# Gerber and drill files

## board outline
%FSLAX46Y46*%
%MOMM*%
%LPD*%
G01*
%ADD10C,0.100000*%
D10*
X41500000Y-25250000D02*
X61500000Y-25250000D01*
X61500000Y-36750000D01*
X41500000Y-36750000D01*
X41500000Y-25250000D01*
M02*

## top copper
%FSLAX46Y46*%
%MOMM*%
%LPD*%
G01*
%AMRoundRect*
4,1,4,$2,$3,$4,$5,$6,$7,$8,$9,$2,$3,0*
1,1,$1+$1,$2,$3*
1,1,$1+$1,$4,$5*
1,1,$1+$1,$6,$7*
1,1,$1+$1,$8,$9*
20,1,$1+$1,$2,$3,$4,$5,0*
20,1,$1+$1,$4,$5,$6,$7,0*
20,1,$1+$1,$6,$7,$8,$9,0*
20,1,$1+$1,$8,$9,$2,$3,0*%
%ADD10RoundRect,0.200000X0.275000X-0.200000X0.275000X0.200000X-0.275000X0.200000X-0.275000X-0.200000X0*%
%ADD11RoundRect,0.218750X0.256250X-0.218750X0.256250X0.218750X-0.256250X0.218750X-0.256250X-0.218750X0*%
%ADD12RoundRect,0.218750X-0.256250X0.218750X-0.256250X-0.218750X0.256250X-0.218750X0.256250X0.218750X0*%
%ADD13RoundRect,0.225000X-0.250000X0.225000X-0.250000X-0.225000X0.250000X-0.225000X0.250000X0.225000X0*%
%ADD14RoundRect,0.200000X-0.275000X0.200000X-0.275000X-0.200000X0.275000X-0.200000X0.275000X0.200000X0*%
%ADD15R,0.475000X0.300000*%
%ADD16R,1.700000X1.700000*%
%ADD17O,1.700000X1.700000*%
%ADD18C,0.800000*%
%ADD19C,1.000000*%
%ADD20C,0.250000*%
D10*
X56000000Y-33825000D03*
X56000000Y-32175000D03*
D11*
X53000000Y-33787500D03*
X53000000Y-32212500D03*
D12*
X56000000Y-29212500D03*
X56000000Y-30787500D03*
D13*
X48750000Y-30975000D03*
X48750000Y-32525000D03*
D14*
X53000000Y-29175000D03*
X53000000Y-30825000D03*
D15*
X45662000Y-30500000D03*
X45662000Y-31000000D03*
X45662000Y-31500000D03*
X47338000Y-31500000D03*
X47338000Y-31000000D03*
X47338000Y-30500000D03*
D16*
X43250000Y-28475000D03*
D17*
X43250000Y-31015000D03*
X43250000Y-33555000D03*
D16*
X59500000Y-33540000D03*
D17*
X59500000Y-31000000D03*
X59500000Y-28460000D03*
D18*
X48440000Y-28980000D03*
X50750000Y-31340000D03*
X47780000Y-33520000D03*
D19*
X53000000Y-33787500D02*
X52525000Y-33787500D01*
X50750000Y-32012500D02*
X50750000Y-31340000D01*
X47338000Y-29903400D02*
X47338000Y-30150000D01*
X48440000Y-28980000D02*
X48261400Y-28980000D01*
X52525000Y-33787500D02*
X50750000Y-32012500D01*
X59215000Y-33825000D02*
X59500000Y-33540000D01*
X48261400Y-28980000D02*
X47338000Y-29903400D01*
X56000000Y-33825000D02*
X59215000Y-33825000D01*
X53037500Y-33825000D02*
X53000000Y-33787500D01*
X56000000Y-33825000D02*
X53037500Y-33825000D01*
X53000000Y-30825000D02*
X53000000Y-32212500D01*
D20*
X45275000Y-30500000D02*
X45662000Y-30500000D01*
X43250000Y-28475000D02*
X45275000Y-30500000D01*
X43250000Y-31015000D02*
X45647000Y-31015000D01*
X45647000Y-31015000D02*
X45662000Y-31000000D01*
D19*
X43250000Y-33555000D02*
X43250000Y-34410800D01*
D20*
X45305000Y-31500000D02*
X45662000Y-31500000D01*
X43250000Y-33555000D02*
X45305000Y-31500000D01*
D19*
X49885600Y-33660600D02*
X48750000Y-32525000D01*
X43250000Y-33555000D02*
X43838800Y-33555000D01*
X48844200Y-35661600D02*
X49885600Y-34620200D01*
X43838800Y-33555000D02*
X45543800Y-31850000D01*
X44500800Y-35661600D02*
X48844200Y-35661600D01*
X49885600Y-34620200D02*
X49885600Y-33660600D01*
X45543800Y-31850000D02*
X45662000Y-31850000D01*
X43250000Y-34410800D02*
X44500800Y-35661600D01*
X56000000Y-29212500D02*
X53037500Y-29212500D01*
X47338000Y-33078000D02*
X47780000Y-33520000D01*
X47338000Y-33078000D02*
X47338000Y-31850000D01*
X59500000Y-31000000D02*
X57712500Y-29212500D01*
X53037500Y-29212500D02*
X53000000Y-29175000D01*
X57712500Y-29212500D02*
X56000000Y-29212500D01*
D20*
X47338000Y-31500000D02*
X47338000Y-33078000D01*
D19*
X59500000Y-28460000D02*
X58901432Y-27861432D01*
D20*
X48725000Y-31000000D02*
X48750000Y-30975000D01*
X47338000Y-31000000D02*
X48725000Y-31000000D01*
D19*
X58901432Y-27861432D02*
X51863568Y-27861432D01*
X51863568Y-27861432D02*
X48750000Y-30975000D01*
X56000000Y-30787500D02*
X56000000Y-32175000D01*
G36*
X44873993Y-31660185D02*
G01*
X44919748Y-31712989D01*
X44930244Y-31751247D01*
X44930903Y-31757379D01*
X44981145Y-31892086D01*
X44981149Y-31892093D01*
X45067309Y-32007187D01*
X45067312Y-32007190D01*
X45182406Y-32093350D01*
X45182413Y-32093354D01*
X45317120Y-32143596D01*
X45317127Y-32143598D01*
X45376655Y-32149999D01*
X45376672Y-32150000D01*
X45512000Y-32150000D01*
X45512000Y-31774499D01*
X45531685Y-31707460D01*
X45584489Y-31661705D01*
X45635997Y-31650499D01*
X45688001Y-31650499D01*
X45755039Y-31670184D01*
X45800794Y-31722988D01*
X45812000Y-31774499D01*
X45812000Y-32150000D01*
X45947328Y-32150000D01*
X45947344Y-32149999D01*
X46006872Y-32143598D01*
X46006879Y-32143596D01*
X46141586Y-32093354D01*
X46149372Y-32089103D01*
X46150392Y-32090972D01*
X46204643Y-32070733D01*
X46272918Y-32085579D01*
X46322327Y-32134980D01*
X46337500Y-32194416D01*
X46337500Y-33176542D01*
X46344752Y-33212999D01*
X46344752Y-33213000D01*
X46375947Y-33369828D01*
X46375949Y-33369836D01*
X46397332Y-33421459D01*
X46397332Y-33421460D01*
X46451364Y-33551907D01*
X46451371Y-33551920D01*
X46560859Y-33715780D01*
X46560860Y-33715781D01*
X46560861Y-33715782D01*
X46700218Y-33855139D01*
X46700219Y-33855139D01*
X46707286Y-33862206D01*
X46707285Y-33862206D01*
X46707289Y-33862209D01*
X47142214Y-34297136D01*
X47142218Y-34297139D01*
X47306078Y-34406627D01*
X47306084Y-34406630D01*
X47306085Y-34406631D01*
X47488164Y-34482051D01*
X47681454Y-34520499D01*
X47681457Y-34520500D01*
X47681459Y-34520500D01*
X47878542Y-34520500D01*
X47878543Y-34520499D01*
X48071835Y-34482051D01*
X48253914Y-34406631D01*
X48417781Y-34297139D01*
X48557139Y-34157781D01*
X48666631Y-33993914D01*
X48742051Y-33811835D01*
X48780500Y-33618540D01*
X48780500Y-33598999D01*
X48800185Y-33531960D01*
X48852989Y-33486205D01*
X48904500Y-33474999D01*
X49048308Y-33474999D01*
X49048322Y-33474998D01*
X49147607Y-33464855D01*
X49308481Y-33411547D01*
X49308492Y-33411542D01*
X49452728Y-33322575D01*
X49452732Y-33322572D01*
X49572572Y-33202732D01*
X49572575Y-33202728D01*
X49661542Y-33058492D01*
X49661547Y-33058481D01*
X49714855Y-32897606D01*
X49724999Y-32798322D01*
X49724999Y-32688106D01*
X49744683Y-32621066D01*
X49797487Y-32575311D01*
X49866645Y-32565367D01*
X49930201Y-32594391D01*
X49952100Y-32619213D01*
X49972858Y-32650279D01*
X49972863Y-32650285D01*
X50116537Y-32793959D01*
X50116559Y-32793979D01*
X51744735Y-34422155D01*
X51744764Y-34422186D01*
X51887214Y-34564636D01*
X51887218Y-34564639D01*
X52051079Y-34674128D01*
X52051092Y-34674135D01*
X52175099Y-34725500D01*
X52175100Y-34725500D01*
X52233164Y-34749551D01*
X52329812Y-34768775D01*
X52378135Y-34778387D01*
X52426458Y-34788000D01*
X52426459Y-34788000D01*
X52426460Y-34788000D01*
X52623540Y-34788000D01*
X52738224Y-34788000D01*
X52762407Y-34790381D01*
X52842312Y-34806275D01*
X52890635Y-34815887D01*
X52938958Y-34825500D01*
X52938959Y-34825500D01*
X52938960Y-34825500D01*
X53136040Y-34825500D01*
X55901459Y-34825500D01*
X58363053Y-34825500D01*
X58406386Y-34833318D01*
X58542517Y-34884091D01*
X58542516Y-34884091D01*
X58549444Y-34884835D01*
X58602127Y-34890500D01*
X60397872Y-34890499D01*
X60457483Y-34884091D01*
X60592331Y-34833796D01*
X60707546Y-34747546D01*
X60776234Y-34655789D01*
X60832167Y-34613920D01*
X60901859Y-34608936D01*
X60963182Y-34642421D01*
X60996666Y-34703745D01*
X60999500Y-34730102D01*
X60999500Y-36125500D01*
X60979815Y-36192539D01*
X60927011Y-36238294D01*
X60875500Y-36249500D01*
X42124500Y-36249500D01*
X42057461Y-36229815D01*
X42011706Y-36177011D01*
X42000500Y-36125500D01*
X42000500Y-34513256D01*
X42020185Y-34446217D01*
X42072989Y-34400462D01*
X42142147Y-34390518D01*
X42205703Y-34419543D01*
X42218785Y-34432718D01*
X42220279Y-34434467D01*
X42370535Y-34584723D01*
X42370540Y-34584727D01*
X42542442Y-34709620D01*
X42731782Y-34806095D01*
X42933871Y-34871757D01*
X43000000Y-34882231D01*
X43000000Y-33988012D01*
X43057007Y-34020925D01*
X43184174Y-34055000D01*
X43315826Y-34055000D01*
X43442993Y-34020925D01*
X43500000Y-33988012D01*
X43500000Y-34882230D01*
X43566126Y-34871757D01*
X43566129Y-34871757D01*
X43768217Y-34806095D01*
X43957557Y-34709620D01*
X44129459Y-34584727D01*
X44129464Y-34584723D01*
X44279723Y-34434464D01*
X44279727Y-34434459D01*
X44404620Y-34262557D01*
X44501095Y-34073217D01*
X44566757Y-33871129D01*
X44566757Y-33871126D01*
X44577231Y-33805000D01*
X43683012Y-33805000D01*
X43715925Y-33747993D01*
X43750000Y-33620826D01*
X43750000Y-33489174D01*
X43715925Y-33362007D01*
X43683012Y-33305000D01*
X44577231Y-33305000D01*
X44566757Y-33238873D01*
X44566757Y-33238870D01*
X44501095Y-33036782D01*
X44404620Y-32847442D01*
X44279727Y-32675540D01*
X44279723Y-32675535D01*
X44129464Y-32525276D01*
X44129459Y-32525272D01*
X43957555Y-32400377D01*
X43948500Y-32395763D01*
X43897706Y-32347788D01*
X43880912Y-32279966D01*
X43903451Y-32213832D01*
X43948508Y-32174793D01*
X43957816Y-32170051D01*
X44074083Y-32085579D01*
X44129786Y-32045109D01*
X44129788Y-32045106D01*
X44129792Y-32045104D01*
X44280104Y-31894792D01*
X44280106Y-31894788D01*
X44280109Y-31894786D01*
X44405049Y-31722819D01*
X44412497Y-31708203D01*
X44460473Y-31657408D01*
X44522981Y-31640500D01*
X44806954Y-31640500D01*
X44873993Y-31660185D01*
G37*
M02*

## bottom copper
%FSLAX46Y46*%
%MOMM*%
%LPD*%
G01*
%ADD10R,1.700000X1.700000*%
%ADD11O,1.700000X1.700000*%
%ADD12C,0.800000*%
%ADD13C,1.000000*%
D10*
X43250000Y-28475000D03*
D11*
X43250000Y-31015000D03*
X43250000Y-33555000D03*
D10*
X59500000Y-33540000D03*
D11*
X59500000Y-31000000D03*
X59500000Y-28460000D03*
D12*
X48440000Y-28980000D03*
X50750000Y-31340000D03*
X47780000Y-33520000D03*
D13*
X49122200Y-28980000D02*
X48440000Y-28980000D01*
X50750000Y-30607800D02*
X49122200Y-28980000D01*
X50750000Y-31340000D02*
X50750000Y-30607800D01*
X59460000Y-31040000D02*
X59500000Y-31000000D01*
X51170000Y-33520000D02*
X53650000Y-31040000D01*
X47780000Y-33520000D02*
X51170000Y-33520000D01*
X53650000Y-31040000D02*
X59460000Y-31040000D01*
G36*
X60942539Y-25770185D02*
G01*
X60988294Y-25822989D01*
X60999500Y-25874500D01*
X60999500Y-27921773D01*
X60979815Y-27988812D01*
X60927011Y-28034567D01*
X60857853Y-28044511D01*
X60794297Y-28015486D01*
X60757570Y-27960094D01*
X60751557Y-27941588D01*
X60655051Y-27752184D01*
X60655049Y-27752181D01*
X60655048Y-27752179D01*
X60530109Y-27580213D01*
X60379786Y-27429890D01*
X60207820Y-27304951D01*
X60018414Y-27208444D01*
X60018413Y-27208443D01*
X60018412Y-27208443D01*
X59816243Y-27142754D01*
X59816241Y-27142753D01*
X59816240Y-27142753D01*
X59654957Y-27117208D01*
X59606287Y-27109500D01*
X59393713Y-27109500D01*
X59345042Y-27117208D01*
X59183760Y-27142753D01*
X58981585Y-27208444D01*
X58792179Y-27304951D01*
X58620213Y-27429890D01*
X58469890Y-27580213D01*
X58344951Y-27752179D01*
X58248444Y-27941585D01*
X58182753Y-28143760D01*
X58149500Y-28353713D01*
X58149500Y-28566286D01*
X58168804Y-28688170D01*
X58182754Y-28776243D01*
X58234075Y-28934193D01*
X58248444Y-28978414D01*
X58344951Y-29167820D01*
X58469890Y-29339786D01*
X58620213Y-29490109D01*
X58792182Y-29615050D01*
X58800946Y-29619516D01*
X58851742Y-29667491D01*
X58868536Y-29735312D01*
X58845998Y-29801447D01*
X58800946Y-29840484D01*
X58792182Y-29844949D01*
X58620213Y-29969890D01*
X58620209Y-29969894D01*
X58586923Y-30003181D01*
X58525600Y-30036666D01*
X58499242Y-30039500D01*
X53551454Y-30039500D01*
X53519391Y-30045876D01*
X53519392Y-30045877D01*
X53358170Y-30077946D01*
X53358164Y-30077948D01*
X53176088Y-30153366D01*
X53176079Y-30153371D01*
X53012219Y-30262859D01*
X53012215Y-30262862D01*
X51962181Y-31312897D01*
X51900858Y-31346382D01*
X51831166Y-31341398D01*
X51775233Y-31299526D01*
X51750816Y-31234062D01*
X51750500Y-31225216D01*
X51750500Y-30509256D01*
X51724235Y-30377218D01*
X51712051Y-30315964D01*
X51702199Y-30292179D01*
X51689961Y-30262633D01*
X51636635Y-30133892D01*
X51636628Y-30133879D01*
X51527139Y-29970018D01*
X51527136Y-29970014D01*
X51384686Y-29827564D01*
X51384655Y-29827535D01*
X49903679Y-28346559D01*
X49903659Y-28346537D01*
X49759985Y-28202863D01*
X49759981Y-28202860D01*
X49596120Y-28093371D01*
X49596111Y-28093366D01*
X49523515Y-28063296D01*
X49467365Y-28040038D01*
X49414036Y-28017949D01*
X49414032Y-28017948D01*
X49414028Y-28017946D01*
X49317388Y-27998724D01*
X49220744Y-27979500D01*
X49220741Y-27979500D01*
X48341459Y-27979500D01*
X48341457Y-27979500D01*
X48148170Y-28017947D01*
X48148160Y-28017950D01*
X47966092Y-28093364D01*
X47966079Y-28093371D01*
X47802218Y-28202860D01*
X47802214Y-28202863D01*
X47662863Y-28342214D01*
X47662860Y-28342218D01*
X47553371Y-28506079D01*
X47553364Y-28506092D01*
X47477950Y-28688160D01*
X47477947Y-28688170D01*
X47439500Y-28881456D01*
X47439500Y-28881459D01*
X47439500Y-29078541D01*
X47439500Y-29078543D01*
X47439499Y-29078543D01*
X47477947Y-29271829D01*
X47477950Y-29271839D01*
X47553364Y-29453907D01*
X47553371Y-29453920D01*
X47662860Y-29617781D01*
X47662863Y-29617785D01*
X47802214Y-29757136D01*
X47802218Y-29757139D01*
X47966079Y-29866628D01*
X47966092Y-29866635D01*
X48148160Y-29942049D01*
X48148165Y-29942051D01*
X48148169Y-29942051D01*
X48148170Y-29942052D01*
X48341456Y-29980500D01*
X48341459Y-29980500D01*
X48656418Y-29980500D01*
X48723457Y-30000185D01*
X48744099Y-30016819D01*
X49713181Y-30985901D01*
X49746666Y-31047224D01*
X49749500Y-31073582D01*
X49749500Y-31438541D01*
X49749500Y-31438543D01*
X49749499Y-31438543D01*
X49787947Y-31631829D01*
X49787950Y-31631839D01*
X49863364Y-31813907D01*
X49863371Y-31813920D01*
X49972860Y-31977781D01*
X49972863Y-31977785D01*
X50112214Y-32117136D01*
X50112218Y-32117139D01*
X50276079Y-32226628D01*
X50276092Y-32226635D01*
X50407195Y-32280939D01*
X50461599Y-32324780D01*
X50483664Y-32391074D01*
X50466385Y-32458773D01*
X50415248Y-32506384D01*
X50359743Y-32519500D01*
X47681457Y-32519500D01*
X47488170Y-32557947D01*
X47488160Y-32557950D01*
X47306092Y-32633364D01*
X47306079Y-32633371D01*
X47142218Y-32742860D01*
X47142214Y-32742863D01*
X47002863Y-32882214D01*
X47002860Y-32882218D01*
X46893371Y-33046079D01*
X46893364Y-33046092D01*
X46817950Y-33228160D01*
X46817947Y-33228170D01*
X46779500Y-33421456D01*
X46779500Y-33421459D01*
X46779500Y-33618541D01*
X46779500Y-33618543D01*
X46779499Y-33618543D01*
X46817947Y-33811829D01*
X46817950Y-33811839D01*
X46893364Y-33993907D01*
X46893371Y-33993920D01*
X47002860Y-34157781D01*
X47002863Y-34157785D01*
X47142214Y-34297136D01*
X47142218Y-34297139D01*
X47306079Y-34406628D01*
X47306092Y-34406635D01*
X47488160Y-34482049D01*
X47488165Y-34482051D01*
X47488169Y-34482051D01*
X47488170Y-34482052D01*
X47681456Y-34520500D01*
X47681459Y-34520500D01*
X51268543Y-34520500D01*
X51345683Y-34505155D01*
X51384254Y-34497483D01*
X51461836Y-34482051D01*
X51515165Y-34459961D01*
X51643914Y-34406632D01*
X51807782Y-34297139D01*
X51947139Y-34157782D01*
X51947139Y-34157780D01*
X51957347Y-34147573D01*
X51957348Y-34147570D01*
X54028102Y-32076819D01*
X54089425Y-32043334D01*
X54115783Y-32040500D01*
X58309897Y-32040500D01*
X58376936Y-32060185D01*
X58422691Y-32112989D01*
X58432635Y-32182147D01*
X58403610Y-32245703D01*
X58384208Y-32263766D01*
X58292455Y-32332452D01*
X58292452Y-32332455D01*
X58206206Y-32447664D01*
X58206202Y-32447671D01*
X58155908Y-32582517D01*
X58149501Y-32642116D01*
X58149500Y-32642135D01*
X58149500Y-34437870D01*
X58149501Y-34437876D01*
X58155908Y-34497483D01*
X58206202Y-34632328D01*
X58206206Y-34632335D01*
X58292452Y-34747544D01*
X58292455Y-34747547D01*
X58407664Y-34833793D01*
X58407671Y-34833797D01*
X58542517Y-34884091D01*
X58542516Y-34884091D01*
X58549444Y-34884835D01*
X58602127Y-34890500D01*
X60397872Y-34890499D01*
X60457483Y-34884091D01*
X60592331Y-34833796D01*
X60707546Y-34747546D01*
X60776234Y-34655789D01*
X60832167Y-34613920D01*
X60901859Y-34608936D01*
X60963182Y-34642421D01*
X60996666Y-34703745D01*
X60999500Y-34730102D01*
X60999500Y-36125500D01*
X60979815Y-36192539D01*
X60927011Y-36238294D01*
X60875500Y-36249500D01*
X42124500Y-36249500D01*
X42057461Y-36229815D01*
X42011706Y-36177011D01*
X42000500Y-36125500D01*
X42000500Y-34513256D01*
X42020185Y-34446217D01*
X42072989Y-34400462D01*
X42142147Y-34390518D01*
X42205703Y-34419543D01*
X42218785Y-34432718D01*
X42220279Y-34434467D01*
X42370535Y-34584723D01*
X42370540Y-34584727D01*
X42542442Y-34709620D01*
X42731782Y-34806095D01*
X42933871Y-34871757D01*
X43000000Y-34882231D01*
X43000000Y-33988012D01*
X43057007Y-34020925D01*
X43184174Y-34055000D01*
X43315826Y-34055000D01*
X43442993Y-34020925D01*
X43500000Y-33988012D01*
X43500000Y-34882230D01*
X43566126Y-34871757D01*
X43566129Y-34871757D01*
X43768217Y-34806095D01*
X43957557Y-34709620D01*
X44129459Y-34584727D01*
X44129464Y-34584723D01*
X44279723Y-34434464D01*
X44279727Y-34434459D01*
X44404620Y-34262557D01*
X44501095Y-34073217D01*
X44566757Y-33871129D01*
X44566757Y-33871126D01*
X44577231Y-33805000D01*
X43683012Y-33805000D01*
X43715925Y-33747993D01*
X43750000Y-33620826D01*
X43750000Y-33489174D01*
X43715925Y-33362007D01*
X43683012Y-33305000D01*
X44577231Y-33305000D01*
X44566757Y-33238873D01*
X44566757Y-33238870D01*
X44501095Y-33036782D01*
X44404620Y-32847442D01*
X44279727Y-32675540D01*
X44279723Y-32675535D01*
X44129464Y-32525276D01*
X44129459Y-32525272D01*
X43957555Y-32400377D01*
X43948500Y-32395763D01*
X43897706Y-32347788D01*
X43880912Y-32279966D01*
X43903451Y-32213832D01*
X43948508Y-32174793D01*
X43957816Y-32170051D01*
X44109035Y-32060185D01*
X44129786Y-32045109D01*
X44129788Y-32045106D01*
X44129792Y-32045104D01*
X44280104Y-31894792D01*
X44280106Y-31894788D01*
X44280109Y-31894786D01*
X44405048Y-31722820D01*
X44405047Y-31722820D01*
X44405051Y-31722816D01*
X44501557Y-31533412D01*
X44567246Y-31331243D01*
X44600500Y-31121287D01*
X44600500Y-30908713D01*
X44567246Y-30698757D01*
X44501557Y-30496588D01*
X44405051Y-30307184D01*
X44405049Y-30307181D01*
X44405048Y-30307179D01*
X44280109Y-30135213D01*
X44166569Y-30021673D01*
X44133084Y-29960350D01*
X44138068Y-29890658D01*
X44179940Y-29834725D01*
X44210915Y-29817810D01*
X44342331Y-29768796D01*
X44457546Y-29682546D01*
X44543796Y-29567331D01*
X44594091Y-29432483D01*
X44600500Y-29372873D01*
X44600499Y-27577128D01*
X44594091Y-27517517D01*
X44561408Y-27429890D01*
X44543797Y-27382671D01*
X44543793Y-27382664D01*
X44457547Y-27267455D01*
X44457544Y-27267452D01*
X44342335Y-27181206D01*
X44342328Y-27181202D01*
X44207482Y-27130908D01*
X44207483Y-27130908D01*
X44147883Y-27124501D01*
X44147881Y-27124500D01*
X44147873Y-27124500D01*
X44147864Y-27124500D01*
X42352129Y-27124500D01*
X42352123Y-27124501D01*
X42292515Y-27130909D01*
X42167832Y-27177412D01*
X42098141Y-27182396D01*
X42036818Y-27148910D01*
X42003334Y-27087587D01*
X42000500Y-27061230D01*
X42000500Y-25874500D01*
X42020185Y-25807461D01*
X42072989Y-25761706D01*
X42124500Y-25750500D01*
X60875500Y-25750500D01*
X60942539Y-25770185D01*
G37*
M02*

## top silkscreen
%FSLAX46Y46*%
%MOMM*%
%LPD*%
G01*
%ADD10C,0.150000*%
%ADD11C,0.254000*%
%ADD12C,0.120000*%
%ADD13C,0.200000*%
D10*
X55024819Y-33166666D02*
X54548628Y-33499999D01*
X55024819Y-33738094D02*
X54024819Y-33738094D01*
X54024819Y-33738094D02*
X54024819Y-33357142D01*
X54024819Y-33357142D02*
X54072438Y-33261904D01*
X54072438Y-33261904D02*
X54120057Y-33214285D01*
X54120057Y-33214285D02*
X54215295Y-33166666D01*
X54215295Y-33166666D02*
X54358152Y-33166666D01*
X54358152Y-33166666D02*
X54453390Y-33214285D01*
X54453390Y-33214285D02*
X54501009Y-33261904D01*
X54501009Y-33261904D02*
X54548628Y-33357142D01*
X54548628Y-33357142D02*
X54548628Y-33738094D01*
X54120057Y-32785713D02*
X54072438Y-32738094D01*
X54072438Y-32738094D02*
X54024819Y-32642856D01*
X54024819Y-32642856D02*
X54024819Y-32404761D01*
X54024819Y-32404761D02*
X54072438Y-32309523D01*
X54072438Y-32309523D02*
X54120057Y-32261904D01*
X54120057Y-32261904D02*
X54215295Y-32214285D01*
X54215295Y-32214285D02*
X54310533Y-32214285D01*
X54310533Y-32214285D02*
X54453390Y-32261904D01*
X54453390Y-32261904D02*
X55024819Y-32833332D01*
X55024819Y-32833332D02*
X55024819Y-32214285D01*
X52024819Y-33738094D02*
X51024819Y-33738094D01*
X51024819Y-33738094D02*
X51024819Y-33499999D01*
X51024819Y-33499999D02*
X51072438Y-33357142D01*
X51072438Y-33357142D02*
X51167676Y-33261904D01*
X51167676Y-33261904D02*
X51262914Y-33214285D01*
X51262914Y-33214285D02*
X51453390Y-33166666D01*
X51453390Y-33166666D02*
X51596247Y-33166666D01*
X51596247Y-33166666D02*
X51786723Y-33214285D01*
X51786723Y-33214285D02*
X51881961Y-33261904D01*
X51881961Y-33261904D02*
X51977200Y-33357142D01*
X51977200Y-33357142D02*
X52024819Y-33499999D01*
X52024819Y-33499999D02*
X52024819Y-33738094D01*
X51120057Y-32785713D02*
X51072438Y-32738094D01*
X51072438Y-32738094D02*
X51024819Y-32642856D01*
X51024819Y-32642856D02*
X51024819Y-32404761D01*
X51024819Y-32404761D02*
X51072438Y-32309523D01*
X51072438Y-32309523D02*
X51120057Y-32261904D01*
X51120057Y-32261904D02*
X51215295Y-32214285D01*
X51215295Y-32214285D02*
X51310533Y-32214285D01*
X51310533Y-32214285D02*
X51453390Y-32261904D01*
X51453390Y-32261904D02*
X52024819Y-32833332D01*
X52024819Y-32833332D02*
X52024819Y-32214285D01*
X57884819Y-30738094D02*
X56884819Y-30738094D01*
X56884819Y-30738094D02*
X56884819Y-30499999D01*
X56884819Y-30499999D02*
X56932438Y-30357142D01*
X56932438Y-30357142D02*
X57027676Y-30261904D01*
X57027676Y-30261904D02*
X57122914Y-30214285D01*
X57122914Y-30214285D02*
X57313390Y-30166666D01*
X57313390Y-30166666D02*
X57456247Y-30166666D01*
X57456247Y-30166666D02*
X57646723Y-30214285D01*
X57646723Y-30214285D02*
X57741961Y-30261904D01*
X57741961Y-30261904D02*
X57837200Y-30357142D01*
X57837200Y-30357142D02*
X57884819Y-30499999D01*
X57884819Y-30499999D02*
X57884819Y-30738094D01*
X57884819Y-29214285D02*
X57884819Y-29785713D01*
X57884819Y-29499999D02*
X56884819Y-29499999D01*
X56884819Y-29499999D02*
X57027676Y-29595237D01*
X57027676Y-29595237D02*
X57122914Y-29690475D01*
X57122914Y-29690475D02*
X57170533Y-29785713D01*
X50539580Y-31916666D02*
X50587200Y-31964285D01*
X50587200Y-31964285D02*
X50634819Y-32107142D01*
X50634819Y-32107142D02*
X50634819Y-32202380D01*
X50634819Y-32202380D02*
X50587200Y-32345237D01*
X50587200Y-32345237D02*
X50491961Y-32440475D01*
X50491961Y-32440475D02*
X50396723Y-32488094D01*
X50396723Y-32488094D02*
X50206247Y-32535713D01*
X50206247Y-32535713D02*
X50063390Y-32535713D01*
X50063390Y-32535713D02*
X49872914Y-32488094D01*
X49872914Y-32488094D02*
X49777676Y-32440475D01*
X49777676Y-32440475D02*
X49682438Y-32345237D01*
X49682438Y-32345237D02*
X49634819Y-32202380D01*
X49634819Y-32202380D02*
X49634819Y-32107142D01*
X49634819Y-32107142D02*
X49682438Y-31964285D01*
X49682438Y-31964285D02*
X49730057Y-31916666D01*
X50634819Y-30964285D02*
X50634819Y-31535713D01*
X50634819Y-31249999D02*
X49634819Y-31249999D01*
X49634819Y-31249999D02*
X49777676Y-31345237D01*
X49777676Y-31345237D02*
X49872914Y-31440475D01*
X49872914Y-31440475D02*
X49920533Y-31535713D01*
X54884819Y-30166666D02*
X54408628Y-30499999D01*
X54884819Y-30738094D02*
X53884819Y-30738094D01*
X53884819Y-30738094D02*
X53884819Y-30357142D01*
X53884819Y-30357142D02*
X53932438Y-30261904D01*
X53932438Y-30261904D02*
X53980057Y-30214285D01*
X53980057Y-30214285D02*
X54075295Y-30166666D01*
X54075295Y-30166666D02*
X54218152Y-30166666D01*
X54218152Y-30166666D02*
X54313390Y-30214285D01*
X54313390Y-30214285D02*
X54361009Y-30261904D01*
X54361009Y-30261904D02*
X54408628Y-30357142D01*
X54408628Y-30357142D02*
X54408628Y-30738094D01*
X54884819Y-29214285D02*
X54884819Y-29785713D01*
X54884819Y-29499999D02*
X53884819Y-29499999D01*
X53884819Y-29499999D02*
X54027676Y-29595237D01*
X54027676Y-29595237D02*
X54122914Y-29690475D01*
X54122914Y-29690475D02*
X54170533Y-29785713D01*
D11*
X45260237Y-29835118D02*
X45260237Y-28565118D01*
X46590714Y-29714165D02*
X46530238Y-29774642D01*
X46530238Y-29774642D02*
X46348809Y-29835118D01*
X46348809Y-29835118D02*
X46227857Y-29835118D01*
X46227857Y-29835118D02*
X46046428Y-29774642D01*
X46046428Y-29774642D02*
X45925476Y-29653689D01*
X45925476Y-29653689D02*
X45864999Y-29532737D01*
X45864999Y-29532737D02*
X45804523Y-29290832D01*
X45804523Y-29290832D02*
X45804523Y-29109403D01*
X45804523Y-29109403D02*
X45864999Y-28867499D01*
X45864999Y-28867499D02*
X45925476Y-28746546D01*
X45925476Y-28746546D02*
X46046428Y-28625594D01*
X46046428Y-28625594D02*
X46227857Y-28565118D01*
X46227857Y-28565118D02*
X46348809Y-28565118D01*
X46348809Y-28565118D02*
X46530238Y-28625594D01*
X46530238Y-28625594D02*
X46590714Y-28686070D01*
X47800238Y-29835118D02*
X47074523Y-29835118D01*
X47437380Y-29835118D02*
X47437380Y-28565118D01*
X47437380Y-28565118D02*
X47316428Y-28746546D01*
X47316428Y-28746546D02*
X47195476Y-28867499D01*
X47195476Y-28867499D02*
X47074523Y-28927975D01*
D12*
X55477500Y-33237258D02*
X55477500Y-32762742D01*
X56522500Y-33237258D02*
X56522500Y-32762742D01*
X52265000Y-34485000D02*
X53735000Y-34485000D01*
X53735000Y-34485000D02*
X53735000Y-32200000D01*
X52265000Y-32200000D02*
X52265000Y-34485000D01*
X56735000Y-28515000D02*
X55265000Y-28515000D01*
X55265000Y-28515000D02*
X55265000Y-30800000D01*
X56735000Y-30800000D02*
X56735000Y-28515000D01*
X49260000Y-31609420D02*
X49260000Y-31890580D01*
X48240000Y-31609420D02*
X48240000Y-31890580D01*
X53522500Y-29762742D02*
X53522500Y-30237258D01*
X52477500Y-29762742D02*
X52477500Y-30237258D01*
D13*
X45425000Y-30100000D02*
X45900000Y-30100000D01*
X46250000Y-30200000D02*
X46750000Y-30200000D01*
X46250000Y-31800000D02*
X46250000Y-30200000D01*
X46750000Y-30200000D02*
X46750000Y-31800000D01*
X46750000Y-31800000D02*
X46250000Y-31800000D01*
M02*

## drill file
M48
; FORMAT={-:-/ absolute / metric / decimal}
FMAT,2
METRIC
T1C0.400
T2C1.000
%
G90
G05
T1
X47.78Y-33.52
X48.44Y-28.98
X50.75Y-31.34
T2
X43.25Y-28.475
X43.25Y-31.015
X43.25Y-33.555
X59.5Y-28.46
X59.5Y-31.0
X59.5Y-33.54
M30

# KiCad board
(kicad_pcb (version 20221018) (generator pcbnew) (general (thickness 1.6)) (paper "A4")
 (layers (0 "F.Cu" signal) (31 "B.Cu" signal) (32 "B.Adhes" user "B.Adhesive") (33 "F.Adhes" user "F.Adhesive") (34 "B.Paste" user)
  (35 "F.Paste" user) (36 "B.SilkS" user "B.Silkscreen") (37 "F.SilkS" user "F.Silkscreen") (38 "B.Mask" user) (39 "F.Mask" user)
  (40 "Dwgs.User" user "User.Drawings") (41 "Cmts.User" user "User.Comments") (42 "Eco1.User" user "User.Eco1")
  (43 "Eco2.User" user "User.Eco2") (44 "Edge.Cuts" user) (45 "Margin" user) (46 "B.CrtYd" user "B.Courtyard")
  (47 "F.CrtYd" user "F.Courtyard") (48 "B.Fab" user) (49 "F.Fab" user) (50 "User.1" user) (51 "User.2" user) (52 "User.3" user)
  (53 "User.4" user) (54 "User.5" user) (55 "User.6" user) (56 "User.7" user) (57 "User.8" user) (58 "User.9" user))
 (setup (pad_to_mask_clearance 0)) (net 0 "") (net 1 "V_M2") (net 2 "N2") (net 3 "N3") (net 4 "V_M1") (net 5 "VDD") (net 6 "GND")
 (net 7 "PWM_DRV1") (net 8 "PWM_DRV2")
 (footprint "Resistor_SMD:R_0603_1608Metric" (layer "F.Cu") (at 56 33 90)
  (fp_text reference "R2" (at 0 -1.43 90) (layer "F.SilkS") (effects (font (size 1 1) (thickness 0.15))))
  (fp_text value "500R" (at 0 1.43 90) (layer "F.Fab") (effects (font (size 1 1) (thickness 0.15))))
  (fp_line (start -0.237258 -0.5225) (end 0.237258 -0.5225) (stroke (width 0.12) (type solid)) (layer "F.SilkS"))
  (fp_line (start -0.237258 0.5225) (end 0.237258 0.5225) (stroke (width 0.12) (type solid)) (layer "F.SilkS"))
  (pad "1" smd roundrect (at -0.825 0 90) (size 0.8 0.95) (layers "F.Cu" "F.Paste" "F.Mask") (roundrect_rratio 0.25) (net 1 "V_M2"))
  (pad "2" smd roundrect (at 0.825 0 90) (size 0.8 0.95) (layers "F.Cu" "F.Paste" "F.Mask") (roundrect_rratio 0.25) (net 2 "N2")))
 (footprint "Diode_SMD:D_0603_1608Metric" (layer "F.Cu") (at 53 33 90)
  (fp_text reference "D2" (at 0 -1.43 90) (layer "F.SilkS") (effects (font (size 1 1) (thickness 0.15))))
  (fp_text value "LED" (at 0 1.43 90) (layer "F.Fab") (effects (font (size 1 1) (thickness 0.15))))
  (fp_line (start -1.485 -0.735) (end -1.485 0.735) (stroke (width 0.12) (type solid)) (layer "F.SilkS"))
  (fp_line (start -1.485 0.735) (end 0.8 0.735) (stroke (width 0.12) (type solid)) (layer "F.SilkS"))
  (fp_line (start 0.8 -0.735) (end -1.485 -0.735) (stroke (width 0.12) (type solid)) (layer "F.SilkS"))
  (pad "1" smd roundrect (at -0.7875 0 90) (size 0.875 0.95) (layers "F.Cu" "F.Paste" "F.Mask") (roundrect_rratio 0.25) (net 1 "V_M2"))
  (pad "2" smd roundrect (at 0.7875 0 90) (size 0.875 0.95) (layers "F.Cu" "F.Paste" "F.Mask") (roundrect_rratio 0.25) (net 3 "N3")))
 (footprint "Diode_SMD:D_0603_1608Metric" (layer "F.Cu") (at 56 30 -90)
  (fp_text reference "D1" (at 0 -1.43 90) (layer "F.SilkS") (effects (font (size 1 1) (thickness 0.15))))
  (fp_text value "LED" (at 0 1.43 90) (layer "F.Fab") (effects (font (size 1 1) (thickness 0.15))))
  (fp_line (start -1.485 -0.735) (end -1.485 0.735) (stroke (width 0.12) (type solid)) (layer "F.SilkS"))
  (fp_line (start -1.485 0.735) (end 0.8 0.735) (stroke (width 0.12) (type solid)) (layer "F.SilkS"))
  (fp_line (start 0.8 -0.735) (end -1.485 -0.735) (stroke (width 0.12) (type solid)) (layer "F.SilkS"))
  (pad "1" smd roundrect (at -0.7875 0 270) (size 0.875 0.95) (layers "F.Cu" "F.Paste" "F.Mask") (roundrect_rratio 0.25) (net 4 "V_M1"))
  (pad "2" smd roundrect (at 0.7875 0 270) (size 0.875 0.95) (layers "F.Cu" "F.Paste" "F.Mask") (roundrect_rratio 0.25) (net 2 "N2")))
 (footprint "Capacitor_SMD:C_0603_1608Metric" (layer "F.Cu") (at 48.75 31.75 -90)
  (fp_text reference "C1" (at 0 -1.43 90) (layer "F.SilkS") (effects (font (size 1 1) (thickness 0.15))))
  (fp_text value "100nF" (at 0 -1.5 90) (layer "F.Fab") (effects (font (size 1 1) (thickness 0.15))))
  (fp_line (start -0.14058 -0.51) (end 0.14058 -0.51) (stroke (width 0.12) (type solid)) (layer "F.SilkS"))
  (fp_line (start -0.14058 0.51) (end 0.14058 0.51) (stroke (width 0.12) (type solid)) (layer "F.SilkS"))
  (pad "1" smd roundrect (at -0.775 0 270) (size 0.9 0.95) (layers "F.Cu" "F.Paste" "F.Mask") (roundrect_rratio 0.25) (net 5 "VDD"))
  (pad "2" smd roundrect (at 0.775 0 270) (size 0.9 0.95) (layers "F.Cu" "F.Paste" "F.Mask") (roundrect_rratio 0.25) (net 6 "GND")))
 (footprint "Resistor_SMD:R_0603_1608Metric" (layer "F.Cu") (at 53 30 -90)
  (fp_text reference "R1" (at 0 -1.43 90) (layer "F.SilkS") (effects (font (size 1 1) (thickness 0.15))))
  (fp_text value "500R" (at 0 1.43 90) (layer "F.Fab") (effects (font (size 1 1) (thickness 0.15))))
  (fp_line (start -0.237258 -0.5225) (end 0.237258 -0.5225) (stroke (width 0.12) (type solid)) (layer "F.SilkS"))
  (fp_line (start -0.237258 0.5225) (end 0.237258 0.5225) (stroke (width 0.12) (type solid)) (layer "F.SilkS"))
  (pad "1" smd roundrect (at -0.825 0 270) (size 0.8 0.95) (layers "F.Cu" "F.Paste" "F.Mask") (roundrect_rratio 0.25) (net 4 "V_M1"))
  (pad "2" smd roundrect (at 0.825 0 270) (size 0.8 0.95) (layers "F.Cu" "F.Paste" "F.Mask") (roundrect_rratio 0.25) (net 3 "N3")))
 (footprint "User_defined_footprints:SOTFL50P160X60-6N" (layer "F.Cu") (at 46.5 31)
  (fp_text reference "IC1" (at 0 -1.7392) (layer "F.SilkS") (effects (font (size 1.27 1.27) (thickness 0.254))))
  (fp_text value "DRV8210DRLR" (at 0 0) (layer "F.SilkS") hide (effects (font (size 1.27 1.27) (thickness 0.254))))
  (fp_line (start -1.075 -0.9) (end -0.6 -0.9) (stroke (width 0.2) (type solid)) (layer "F.SilkS"))
  (fp_line (start -0.25 -0.8) (end 0.25 -0.8) (stroke (width 0.2) (type solid)) (layer "F.SilkS"))
  (fp_line (start -0.25 0.8) (end -0.25 -0.8) (stroke (width 0.2) (type solid)) (layer "F.SilkS"))
  (fp_line (start 0.25 -0.8) (end 0.25 0.8) (stroke (width 0.2) (type solid)) (layer "F.SilkS"))
  (fp_line (start 0.25 0.8) (end -0.25 0.8) (stroke (width 0.2) (type solid)) (layer "F.SilkS"))
  (pad "1" smd rect (at -0.838 -0.5 90) (size 0.3 0.475) (layers "F.Cu" "F.Paste" "F.Mask") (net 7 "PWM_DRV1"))
  (pad "2" smd rect (at -0.838 0 90) (size 0.3 0.475) (layers "F.Cu" "F.Paste" "F.Mask") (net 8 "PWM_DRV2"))
  (pad "3" smd rect (at -0.838 0.5 90) (size 0.3 0.475) (layers "F.Cu" "F.Paste" "F.Mask") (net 6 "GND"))
  (pad "4" smd rect (at 0.838 0.5 90) (size 0.3 0.475) (layers "F.Cu" "F.Paste" "F.Mask") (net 4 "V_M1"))
  (pad "5" smd rect (at 0.838 0 90) (size 0.3 0.475) (layers "F.Cu" "F.Paste" "F.Mask") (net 5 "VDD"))
  (pad "6" smd rect (at 0.838 -0.5 90) (size 0.3 0.475) (layers "F.Cu" "F.Paste" "F.Mask") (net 1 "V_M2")))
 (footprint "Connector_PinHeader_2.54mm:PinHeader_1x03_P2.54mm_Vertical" (layer "B.Cu") (at 43.25 28.475 180)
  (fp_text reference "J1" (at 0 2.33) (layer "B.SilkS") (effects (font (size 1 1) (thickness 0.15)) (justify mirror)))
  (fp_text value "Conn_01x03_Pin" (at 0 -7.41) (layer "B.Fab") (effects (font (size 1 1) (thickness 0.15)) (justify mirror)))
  (pad "1" thru_hole rect (at 0 0 180) (size 1.7 1.7) (drill 1) (layers "*.Cu" "*.Mask") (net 7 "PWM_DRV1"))
  (pad "2" thru_hole oval (at 0 -2.54 180) (size 1.7 1.7) (drill 1) (layers "*.Cu" "*.Mask") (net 8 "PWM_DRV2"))
  (pad "3" thru_hole oval (at 0 -5.08 180) (size 1.7 1.7) (drill 1) (layers "*.Cu" "*.Mask") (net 6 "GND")))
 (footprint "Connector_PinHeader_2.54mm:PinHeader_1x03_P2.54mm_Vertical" (layer "B.Cu") (at 59.5 33.54)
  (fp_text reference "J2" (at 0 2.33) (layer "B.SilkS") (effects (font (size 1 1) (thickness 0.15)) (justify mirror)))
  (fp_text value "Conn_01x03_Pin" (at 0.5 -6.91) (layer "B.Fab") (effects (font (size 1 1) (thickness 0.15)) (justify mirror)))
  (pad "1" thru_hole rect (at 0 0) (size 1.7 1.7) (drill 1) (layers "*.Cu" "*.Mask") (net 1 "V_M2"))
  (pad "2" thru_hole oval (at 0 -2.54) (size 1.7 1.7) (drill 1) (layers "*.Cu" "*.Mask") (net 4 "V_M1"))
  (pad "3" thru_hole oval (at 0 -5.08) (size 1.7 1.7) (drill 1) (layers "*.Cu" "*.Mask") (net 5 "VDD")))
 (gr_rect (start 41.5 25.25) (end 61.5 36.75) (stroke (width 0.1) (type default)) (fill none) (layer "Edge.Cuts"))
 (segment (start 53 33.7875) (end 52.525 33.7875) (width 1) (layer "F.Cu") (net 1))
 (segment (start 50.75 32.0125) (end 50.75 31.34) (width 1) (layer "F.Cu") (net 1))
 (segment (start 47.338 29.9034) (end 47.338 30.15) (width 1) (layer "F.Cu") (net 1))
 (segment (start 48.44 28.98) (end 48.2614 28.98) (width 1) (layer "F.Cu") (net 1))
 (segment (start 52.525 33.7875) (end 50.75 32.0125) (width 1) (layer "F.Cu") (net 1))
 (segment (start 59.215 33.825) (end 59.5 33.54) (width 1) (layer "F.Cu") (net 1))
 (segment (start 48.2614 28.98) (end 47.338 29.9034) (width 1) (layer "F.Cu") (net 1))
 (segment (start 56 33.825) (end 59.215 33.825) (width 1) (layer "F.Cu") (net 1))
 (segment (start 53.0375 33.825) (end 53 33.7875) (width 1) (layer "F.Cu") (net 1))
 (segment (start 56 33.825) (end 53.0375 33.825) (width 1) (layer "F.Cu") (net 1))
 (via (at 48.44 28.98) (size 0.8) (drill 0.4) (layers "F.Cu" "B.Cu") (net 1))
 (via (at 50.75 31.34) (size 0.8) (drill 0.4) (layers "F.Cu" "B.Cu") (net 1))
 (segment (start 49.1222 28.98) (end 48.44 28.98) (width 1) (layer "B.Cu") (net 1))
 (segment (start 50.75 30.6078) (end 49.1222 28.98) (width 1) (layer "B.Cu") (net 1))
 (segment (start 50.75 31.34) (end 50.75 30.6078) (width 1) (layer "B.Cu") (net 1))
 (segment (start 53 30.825) (end 53 32.2125) (width 1) (layer "F.Cu") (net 3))
 (segment (start 45.275 30.5) (end 45.662 30.5) (width 0.25) (layer "F.Cu") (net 7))
 (segment (start 43.25 28.475) (end 45.275 30.5) (width 0.25) (layer "F.Cu") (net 7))
 (segment (start 43.25 31.015) (end 45.647 31.015) (width 0.25) (layer "F.Cu") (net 8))
 (segment (start 45.647 31.015) (end 45.662 31) (width 0.25) (layer "F.Cu") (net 8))
 (segment (start 43.25 33.555) (end 43.25 34.4108) (width 1) (layer "F.Cu") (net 6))
 (segment (start 45.305 31.5) (end 45.662 31.5) (width 0.25) (layer "F.Cu") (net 6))
 (segment (start 43.25 33.555) (end 45.305 31.5) (width 0.25) (layer "F.Cu") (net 6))
 (segment (start 49.8856 33.6606) (end 48.75 32.525) (width 1) (layer "F.Cu") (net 6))
 (segment (start 43.25 33.555) (end 43.8388 33.555) (width 1) (layer "F.Cu") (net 6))
 (segment (start 48.8442 35.6616) (end 49.8856 34.6202) (width 1) (layer "F.Cu") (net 6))
 (segment (start 43.8388 33.555) (end 45.5438 31.85) (width 1) (layer "F.Cu") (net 6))
 (segment (start 44.5008 35.6616) (end 48.8442 35.6616) (width 1) (layer "F.Cu") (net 6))
 (segment (start 49.8856 34.6202) (end 49.8856 33.6606) (width 1) (layer "F.Cu") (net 6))
 (segment (start 45.5438 31.85) (end 45.662 31.85) (width 1) (layer "F.Cu") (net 6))
 (segment (start 43.25 34.4108) (end 44.5008 35.6616) (width 1) (layer "F.Cu") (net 6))
 (segment (start 56 29.2125) (end 53.0375 29.2125) (width 1) (layer "F.Cu") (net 4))
 (segment (start 47.338 33.078) (end 47.78 33.52) (width 1) (layer "F.Cu") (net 4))
 (segment (start 47.338 33.078) (end 47.338 31.85) (width 1) (layer "F.Cu") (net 4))
 (segment (start 59.5 31) (end 57.7125 29.2125) (width 1) (layer "F.Cu") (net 4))
 (segment (start 53.0375 29.2125) (end 53 29.175) (width 1) (layer "F.Cu") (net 4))
 (segment (start 57.7125 29.2125) (end 56 29.2125) (width 1) (layer "F.Cu") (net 4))
 (segment (start 47.338 31.5) (end 47.338 33.078) (width 0.25) (layer "F.Cu") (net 4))
 (via (at 47.78 33.52) (size 0.8) (drill 0.4) (layers "F.Cu" "B.Cu") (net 4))
 (segment (start 59.46 31.04) (end 59.5 31) (width 1) (layer "B.Cu") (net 4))
 (segment (start 51.17 33.52) (end 53.65 31.04) (width 1) (layer "B.Cu") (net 4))
 (segment (start 47.78 33.52) (end 51.17 33.52) (width 1) (layer "B.Cu") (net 4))
 (segment (start 53.65 31.04) (end 59.46 31.04) (width 1) (layer "B.Cu") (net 4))
 (segment (start 59.5 28.46) (end 58.901432 27.861432) (width 1) (layer "F.Cu") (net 5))
 (segment (start 48.725 31) (end 48.75 30.975) (width 0.25) (layer "F.Cu") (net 5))
 (segment (start 47.338 31) (end 48.725 31) (width 0.25) (layer "F.Cu") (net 5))
 (segment (start 58.901432 27.861432) (end 51.863568 27.861432) (width 1) (layer "F.Cu") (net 5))
 (segment (start 51.863568 27.861432) (end 48.75 30.975) (width 1) (layer "F.Cu") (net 5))
 (segment (start 56 30.7875) (end 56 32.175) (width 1) (layer "F.Cu") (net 2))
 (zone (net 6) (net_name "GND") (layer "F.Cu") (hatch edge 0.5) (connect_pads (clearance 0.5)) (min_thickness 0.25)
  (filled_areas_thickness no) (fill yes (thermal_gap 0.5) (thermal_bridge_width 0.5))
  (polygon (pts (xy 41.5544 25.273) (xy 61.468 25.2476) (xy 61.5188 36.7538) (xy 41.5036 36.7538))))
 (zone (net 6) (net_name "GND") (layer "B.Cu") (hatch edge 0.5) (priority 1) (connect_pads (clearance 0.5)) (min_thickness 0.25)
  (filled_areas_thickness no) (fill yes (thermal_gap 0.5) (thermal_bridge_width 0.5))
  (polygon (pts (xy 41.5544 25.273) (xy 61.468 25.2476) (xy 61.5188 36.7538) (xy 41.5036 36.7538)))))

